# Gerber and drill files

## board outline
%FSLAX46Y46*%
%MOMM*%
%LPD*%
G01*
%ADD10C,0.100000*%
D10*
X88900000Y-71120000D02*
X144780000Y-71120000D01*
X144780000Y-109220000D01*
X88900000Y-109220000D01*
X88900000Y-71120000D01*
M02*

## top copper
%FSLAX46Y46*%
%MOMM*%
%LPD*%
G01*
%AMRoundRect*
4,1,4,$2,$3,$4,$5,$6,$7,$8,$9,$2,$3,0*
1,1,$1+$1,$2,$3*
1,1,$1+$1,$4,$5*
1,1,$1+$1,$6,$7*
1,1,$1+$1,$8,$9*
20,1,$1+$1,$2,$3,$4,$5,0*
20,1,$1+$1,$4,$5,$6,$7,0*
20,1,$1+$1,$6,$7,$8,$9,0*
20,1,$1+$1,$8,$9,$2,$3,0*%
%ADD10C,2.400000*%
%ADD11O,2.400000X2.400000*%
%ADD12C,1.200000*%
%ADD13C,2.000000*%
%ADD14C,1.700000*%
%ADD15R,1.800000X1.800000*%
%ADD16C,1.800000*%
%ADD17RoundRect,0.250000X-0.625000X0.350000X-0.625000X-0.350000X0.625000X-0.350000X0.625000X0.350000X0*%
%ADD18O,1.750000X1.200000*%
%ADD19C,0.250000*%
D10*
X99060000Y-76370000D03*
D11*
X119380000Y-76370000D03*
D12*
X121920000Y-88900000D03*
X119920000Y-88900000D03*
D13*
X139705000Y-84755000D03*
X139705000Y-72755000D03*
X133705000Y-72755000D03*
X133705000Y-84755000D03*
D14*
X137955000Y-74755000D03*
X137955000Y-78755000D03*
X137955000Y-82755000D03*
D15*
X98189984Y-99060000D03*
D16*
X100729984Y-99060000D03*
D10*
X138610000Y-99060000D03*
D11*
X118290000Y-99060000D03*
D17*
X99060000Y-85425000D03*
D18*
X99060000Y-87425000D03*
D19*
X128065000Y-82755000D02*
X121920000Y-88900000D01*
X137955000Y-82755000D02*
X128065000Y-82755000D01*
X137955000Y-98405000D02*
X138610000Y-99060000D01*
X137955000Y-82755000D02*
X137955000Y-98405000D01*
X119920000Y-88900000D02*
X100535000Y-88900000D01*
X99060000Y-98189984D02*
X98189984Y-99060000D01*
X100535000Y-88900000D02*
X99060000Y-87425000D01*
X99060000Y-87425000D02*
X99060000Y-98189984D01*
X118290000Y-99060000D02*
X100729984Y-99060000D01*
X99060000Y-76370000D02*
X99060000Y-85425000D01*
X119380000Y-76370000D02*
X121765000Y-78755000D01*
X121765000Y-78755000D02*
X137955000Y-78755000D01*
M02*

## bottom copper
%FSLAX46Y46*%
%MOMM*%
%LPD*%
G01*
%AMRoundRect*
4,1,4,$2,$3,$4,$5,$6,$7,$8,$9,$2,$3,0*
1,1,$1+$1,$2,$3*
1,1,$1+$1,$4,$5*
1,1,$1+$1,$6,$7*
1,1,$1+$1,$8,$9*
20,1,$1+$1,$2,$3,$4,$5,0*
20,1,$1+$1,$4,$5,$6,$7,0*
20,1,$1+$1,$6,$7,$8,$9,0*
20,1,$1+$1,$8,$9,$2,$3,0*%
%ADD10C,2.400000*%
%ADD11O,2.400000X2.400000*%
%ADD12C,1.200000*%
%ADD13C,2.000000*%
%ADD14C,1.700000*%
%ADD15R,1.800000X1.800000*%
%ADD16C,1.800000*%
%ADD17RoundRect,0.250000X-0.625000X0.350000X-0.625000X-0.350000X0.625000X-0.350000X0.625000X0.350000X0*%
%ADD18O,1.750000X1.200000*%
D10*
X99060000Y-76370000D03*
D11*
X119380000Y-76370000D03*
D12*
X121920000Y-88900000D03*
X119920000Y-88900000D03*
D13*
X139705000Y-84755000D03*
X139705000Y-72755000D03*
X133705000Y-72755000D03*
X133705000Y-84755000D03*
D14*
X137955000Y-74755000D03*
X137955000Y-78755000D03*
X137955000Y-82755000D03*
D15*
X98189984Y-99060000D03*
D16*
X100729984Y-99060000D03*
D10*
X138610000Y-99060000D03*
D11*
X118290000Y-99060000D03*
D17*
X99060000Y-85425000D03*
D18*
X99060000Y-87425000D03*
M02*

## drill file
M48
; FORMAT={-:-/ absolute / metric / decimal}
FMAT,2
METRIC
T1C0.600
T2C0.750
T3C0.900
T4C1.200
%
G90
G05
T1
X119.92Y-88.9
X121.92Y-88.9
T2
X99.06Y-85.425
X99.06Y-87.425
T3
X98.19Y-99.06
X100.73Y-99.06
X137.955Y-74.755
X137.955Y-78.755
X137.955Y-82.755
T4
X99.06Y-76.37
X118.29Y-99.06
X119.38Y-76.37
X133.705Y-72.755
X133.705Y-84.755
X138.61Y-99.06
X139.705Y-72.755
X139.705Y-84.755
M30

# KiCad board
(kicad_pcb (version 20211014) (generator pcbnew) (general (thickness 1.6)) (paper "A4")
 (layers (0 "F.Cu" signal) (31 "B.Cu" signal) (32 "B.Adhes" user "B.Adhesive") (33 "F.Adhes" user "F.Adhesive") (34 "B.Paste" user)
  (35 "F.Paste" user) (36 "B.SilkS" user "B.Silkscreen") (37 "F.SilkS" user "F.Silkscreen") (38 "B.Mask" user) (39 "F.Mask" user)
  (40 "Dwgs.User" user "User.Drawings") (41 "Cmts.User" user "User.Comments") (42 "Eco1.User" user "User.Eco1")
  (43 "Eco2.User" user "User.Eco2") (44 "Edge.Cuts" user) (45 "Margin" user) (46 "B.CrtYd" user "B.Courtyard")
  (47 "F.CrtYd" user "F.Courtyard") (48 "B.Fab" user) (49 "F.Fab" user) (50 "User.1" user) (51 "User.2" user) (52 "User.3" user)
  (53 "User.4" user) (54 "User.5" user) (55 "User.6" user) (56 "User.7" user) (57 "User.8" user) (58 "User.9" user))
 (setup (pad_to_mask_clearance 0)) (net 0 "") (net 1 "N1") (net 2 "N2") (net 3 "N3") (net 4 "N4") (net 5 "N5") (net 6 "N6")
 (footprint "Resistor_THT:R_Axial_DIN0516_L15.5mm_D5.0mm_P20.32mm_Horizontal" (layer "F.Cu") (at 99.06 76.37)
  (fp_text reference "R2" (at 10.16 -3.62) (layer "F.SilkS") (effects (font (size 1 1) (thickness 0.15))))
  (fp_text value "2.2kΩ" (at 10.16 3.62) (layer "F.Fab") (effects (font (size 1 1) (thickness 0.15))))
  (pad "1" thru_hole circle (at 0 0) (size 2.4 2.4) (drill 1.2) (layers *.Cu *.Mask) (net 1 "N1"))
  (pad "2" thru_hole oval (at 20.32 0) (size 2.4 2.4) (drill 1.2) (layers *.Cu *.Mask) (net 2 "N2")))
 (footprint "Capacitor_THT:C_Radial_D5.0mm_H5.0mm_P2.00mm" (layer "F.Cu") (at 121.92 88.9 180)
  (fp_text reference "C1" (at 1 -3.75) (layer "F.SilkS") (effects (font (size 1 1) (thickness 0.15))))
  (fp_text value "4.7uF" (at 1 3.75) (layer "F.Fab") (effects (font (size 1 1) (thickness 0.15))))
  (pad "1" thru_hole circle (at 0 0 180) (size 1.2 1.2) (drill 0.6) (layers *.Cu *.Mask) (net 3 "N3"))
  (pad "2" thru_hole circle (at 2 0 180) (size 1.2 1.2) (drill 0.6) (layers *.Cu *.Mask) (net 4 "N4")))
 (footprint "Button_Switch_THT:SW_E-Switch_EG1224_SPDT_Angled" (layer "F.Cu") (at 137.955 74.755 -90)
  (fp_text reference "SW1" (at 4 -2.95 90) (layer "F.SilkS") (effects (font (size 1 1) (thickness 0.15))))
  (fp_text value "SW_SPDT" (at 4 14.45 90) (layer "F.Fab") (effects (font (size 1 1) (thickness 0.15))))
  (pad "" thru_hole circle (at 10 -1.75 270) (size 2 2) (drill 1.2) (layers *.Cu *.Mask))
  (pad "" thru_hole circle (at -2 -1.75 270) (size 2 2) (drill 1.2) (layers *.Cu *.Mask))
  (pad "" thru_hole circle (at -2 4.25 270) (size 2 2) (drill 1.2) (layers *.Cu *.Mask))
  (pad "" thru_hole circle (at 10 4.25 270) (size 2 2) (drill 1.2) (layers *.Cu *.Mask))
  (pad "1" thru_hole circle (at 0 0 270) (size 1.7 1.7) (drill 0.9) (layers *.Cu *.Mask) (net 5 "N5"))
  (pad "2" thru_hole circle (at 4 0 270) (size 1.7 1.7) (drill 0.9) (layers *.Cu *.Mask) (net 2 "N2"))
  (pad "3" thru_hole circle (at 8 0 270) (size 1.7 1.7) (drill 0.9) (layers *.Cu *.Mask) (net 3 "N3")))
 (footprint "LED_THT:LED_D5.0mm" (layer "F.Cu") (at 98.189984 99.06)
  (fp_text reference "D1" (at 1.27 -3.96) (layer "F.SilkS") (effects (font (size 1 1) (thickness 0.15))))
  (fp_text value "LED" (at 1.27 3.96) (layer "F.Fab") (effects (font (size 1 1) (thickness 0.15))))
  (pad "1" thru_hole rect (at 0 0) (size 1.8 1.8) (drill 0.9) (layers *.Cu *.Mask) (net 4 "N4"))
  (pad "2" thru_hole circle (at 2.54 0) (size 1.8 1.8) (drill 0.9) (layers *.Cu *.Mask) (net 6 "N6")))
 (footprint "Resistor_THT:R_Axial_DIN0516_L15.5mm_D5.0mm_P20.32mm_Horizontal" (layer "F.Cu") (at 138.61 99.06 180)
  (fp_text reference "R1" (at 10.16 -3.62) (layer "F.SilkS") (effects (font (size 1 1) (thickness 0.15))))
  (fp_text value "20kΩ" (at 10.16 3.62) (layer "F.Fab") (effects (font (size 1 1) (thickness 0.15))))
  (pad "1" thru_hole circle (at 0 0 180) (size 2.4 2.4) (drill 1.2) (layers *.Cu *.Mask) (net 3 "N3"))
  (pad "2" thru_hole oval (at 20.32 0 180) (size 2.4 2.4) (drill 1.2) (layers *.Cu *.Mask) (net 6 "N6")))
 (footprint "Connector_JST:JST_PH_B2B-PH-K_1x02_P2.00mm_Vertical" (layer "F.Cu") (at 99.06 85.425 -90)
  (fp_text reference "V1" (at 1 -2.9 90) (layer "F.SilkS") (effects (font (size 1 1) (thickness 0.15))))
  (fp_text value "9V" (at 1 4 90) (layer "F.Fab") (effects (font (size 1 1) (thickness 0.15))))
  (pad "1" thru_hole roundrect (at 0 0 270) (size 1.2 1.75) (drill 0.75) (layers *.Cu *.Mask) (roundrect_rratio 0.208333) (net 1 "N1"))
  (pad "2" thru_hole oval (at 2 0 270) (size 1.2 1.75) (drill 0.75) (layers *.Cu *.Mask) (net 4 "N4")))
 (gr_rect (start 144.78 109.22) (end 88.9 71.12) (layer "Edge.Cuts") (width 0.1) (fill none))
 (segment (start 128.065 82.755) (end 121.92 88.9) (width 0.25) (layer "F.Cu") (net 3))
 (segment (start 137.955 82.755) (end 128.065 82.755) (width 0.25) (layer "F.Cu") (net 3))
 (segment (start 137.955 98.405) (end 138.61 99.06) (width 0.25) (layer "F.Cu") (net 3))
 (segment (start 137.955 82.755) (end 137.955 98.405) (width 0.25) (layer "F.Cu") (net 3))
 (segment (start 119.92 88.9) (end 100.535 88.9) (width 0.25) (layer "F.Cu") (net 4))
 (segment (start 99.06 98.189984) (end 98.189984 99.06) (width 0.25) (layer "F.Cu") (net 4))
 (segment (start 100.535 88.9) (end 99.06 87.425) (width 0.25) (layer "F.Cu") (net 4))
 (segment (start 99.06 87.425) (end 99.06 98.189984) (width 0.25) (layer "F.Cu") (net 4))
 (segment (start 118.29 99.06) (end 100.729984 99.06) (width 0.25) (layer "F.Cu") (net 6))
 (segment (start 99.06 76.37) (end 99.06 85.425) (width 0.25) (layer "F.Cu") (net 1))
 (segment (start 119.38 76.37) (end 121.765 78.755) (width 0.25) (layer "F.Cu") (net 2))
 (segment (start 121.765 78.755) (end 137.955 78.755) (width 0.25) (layer "F.Cu") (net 2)))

